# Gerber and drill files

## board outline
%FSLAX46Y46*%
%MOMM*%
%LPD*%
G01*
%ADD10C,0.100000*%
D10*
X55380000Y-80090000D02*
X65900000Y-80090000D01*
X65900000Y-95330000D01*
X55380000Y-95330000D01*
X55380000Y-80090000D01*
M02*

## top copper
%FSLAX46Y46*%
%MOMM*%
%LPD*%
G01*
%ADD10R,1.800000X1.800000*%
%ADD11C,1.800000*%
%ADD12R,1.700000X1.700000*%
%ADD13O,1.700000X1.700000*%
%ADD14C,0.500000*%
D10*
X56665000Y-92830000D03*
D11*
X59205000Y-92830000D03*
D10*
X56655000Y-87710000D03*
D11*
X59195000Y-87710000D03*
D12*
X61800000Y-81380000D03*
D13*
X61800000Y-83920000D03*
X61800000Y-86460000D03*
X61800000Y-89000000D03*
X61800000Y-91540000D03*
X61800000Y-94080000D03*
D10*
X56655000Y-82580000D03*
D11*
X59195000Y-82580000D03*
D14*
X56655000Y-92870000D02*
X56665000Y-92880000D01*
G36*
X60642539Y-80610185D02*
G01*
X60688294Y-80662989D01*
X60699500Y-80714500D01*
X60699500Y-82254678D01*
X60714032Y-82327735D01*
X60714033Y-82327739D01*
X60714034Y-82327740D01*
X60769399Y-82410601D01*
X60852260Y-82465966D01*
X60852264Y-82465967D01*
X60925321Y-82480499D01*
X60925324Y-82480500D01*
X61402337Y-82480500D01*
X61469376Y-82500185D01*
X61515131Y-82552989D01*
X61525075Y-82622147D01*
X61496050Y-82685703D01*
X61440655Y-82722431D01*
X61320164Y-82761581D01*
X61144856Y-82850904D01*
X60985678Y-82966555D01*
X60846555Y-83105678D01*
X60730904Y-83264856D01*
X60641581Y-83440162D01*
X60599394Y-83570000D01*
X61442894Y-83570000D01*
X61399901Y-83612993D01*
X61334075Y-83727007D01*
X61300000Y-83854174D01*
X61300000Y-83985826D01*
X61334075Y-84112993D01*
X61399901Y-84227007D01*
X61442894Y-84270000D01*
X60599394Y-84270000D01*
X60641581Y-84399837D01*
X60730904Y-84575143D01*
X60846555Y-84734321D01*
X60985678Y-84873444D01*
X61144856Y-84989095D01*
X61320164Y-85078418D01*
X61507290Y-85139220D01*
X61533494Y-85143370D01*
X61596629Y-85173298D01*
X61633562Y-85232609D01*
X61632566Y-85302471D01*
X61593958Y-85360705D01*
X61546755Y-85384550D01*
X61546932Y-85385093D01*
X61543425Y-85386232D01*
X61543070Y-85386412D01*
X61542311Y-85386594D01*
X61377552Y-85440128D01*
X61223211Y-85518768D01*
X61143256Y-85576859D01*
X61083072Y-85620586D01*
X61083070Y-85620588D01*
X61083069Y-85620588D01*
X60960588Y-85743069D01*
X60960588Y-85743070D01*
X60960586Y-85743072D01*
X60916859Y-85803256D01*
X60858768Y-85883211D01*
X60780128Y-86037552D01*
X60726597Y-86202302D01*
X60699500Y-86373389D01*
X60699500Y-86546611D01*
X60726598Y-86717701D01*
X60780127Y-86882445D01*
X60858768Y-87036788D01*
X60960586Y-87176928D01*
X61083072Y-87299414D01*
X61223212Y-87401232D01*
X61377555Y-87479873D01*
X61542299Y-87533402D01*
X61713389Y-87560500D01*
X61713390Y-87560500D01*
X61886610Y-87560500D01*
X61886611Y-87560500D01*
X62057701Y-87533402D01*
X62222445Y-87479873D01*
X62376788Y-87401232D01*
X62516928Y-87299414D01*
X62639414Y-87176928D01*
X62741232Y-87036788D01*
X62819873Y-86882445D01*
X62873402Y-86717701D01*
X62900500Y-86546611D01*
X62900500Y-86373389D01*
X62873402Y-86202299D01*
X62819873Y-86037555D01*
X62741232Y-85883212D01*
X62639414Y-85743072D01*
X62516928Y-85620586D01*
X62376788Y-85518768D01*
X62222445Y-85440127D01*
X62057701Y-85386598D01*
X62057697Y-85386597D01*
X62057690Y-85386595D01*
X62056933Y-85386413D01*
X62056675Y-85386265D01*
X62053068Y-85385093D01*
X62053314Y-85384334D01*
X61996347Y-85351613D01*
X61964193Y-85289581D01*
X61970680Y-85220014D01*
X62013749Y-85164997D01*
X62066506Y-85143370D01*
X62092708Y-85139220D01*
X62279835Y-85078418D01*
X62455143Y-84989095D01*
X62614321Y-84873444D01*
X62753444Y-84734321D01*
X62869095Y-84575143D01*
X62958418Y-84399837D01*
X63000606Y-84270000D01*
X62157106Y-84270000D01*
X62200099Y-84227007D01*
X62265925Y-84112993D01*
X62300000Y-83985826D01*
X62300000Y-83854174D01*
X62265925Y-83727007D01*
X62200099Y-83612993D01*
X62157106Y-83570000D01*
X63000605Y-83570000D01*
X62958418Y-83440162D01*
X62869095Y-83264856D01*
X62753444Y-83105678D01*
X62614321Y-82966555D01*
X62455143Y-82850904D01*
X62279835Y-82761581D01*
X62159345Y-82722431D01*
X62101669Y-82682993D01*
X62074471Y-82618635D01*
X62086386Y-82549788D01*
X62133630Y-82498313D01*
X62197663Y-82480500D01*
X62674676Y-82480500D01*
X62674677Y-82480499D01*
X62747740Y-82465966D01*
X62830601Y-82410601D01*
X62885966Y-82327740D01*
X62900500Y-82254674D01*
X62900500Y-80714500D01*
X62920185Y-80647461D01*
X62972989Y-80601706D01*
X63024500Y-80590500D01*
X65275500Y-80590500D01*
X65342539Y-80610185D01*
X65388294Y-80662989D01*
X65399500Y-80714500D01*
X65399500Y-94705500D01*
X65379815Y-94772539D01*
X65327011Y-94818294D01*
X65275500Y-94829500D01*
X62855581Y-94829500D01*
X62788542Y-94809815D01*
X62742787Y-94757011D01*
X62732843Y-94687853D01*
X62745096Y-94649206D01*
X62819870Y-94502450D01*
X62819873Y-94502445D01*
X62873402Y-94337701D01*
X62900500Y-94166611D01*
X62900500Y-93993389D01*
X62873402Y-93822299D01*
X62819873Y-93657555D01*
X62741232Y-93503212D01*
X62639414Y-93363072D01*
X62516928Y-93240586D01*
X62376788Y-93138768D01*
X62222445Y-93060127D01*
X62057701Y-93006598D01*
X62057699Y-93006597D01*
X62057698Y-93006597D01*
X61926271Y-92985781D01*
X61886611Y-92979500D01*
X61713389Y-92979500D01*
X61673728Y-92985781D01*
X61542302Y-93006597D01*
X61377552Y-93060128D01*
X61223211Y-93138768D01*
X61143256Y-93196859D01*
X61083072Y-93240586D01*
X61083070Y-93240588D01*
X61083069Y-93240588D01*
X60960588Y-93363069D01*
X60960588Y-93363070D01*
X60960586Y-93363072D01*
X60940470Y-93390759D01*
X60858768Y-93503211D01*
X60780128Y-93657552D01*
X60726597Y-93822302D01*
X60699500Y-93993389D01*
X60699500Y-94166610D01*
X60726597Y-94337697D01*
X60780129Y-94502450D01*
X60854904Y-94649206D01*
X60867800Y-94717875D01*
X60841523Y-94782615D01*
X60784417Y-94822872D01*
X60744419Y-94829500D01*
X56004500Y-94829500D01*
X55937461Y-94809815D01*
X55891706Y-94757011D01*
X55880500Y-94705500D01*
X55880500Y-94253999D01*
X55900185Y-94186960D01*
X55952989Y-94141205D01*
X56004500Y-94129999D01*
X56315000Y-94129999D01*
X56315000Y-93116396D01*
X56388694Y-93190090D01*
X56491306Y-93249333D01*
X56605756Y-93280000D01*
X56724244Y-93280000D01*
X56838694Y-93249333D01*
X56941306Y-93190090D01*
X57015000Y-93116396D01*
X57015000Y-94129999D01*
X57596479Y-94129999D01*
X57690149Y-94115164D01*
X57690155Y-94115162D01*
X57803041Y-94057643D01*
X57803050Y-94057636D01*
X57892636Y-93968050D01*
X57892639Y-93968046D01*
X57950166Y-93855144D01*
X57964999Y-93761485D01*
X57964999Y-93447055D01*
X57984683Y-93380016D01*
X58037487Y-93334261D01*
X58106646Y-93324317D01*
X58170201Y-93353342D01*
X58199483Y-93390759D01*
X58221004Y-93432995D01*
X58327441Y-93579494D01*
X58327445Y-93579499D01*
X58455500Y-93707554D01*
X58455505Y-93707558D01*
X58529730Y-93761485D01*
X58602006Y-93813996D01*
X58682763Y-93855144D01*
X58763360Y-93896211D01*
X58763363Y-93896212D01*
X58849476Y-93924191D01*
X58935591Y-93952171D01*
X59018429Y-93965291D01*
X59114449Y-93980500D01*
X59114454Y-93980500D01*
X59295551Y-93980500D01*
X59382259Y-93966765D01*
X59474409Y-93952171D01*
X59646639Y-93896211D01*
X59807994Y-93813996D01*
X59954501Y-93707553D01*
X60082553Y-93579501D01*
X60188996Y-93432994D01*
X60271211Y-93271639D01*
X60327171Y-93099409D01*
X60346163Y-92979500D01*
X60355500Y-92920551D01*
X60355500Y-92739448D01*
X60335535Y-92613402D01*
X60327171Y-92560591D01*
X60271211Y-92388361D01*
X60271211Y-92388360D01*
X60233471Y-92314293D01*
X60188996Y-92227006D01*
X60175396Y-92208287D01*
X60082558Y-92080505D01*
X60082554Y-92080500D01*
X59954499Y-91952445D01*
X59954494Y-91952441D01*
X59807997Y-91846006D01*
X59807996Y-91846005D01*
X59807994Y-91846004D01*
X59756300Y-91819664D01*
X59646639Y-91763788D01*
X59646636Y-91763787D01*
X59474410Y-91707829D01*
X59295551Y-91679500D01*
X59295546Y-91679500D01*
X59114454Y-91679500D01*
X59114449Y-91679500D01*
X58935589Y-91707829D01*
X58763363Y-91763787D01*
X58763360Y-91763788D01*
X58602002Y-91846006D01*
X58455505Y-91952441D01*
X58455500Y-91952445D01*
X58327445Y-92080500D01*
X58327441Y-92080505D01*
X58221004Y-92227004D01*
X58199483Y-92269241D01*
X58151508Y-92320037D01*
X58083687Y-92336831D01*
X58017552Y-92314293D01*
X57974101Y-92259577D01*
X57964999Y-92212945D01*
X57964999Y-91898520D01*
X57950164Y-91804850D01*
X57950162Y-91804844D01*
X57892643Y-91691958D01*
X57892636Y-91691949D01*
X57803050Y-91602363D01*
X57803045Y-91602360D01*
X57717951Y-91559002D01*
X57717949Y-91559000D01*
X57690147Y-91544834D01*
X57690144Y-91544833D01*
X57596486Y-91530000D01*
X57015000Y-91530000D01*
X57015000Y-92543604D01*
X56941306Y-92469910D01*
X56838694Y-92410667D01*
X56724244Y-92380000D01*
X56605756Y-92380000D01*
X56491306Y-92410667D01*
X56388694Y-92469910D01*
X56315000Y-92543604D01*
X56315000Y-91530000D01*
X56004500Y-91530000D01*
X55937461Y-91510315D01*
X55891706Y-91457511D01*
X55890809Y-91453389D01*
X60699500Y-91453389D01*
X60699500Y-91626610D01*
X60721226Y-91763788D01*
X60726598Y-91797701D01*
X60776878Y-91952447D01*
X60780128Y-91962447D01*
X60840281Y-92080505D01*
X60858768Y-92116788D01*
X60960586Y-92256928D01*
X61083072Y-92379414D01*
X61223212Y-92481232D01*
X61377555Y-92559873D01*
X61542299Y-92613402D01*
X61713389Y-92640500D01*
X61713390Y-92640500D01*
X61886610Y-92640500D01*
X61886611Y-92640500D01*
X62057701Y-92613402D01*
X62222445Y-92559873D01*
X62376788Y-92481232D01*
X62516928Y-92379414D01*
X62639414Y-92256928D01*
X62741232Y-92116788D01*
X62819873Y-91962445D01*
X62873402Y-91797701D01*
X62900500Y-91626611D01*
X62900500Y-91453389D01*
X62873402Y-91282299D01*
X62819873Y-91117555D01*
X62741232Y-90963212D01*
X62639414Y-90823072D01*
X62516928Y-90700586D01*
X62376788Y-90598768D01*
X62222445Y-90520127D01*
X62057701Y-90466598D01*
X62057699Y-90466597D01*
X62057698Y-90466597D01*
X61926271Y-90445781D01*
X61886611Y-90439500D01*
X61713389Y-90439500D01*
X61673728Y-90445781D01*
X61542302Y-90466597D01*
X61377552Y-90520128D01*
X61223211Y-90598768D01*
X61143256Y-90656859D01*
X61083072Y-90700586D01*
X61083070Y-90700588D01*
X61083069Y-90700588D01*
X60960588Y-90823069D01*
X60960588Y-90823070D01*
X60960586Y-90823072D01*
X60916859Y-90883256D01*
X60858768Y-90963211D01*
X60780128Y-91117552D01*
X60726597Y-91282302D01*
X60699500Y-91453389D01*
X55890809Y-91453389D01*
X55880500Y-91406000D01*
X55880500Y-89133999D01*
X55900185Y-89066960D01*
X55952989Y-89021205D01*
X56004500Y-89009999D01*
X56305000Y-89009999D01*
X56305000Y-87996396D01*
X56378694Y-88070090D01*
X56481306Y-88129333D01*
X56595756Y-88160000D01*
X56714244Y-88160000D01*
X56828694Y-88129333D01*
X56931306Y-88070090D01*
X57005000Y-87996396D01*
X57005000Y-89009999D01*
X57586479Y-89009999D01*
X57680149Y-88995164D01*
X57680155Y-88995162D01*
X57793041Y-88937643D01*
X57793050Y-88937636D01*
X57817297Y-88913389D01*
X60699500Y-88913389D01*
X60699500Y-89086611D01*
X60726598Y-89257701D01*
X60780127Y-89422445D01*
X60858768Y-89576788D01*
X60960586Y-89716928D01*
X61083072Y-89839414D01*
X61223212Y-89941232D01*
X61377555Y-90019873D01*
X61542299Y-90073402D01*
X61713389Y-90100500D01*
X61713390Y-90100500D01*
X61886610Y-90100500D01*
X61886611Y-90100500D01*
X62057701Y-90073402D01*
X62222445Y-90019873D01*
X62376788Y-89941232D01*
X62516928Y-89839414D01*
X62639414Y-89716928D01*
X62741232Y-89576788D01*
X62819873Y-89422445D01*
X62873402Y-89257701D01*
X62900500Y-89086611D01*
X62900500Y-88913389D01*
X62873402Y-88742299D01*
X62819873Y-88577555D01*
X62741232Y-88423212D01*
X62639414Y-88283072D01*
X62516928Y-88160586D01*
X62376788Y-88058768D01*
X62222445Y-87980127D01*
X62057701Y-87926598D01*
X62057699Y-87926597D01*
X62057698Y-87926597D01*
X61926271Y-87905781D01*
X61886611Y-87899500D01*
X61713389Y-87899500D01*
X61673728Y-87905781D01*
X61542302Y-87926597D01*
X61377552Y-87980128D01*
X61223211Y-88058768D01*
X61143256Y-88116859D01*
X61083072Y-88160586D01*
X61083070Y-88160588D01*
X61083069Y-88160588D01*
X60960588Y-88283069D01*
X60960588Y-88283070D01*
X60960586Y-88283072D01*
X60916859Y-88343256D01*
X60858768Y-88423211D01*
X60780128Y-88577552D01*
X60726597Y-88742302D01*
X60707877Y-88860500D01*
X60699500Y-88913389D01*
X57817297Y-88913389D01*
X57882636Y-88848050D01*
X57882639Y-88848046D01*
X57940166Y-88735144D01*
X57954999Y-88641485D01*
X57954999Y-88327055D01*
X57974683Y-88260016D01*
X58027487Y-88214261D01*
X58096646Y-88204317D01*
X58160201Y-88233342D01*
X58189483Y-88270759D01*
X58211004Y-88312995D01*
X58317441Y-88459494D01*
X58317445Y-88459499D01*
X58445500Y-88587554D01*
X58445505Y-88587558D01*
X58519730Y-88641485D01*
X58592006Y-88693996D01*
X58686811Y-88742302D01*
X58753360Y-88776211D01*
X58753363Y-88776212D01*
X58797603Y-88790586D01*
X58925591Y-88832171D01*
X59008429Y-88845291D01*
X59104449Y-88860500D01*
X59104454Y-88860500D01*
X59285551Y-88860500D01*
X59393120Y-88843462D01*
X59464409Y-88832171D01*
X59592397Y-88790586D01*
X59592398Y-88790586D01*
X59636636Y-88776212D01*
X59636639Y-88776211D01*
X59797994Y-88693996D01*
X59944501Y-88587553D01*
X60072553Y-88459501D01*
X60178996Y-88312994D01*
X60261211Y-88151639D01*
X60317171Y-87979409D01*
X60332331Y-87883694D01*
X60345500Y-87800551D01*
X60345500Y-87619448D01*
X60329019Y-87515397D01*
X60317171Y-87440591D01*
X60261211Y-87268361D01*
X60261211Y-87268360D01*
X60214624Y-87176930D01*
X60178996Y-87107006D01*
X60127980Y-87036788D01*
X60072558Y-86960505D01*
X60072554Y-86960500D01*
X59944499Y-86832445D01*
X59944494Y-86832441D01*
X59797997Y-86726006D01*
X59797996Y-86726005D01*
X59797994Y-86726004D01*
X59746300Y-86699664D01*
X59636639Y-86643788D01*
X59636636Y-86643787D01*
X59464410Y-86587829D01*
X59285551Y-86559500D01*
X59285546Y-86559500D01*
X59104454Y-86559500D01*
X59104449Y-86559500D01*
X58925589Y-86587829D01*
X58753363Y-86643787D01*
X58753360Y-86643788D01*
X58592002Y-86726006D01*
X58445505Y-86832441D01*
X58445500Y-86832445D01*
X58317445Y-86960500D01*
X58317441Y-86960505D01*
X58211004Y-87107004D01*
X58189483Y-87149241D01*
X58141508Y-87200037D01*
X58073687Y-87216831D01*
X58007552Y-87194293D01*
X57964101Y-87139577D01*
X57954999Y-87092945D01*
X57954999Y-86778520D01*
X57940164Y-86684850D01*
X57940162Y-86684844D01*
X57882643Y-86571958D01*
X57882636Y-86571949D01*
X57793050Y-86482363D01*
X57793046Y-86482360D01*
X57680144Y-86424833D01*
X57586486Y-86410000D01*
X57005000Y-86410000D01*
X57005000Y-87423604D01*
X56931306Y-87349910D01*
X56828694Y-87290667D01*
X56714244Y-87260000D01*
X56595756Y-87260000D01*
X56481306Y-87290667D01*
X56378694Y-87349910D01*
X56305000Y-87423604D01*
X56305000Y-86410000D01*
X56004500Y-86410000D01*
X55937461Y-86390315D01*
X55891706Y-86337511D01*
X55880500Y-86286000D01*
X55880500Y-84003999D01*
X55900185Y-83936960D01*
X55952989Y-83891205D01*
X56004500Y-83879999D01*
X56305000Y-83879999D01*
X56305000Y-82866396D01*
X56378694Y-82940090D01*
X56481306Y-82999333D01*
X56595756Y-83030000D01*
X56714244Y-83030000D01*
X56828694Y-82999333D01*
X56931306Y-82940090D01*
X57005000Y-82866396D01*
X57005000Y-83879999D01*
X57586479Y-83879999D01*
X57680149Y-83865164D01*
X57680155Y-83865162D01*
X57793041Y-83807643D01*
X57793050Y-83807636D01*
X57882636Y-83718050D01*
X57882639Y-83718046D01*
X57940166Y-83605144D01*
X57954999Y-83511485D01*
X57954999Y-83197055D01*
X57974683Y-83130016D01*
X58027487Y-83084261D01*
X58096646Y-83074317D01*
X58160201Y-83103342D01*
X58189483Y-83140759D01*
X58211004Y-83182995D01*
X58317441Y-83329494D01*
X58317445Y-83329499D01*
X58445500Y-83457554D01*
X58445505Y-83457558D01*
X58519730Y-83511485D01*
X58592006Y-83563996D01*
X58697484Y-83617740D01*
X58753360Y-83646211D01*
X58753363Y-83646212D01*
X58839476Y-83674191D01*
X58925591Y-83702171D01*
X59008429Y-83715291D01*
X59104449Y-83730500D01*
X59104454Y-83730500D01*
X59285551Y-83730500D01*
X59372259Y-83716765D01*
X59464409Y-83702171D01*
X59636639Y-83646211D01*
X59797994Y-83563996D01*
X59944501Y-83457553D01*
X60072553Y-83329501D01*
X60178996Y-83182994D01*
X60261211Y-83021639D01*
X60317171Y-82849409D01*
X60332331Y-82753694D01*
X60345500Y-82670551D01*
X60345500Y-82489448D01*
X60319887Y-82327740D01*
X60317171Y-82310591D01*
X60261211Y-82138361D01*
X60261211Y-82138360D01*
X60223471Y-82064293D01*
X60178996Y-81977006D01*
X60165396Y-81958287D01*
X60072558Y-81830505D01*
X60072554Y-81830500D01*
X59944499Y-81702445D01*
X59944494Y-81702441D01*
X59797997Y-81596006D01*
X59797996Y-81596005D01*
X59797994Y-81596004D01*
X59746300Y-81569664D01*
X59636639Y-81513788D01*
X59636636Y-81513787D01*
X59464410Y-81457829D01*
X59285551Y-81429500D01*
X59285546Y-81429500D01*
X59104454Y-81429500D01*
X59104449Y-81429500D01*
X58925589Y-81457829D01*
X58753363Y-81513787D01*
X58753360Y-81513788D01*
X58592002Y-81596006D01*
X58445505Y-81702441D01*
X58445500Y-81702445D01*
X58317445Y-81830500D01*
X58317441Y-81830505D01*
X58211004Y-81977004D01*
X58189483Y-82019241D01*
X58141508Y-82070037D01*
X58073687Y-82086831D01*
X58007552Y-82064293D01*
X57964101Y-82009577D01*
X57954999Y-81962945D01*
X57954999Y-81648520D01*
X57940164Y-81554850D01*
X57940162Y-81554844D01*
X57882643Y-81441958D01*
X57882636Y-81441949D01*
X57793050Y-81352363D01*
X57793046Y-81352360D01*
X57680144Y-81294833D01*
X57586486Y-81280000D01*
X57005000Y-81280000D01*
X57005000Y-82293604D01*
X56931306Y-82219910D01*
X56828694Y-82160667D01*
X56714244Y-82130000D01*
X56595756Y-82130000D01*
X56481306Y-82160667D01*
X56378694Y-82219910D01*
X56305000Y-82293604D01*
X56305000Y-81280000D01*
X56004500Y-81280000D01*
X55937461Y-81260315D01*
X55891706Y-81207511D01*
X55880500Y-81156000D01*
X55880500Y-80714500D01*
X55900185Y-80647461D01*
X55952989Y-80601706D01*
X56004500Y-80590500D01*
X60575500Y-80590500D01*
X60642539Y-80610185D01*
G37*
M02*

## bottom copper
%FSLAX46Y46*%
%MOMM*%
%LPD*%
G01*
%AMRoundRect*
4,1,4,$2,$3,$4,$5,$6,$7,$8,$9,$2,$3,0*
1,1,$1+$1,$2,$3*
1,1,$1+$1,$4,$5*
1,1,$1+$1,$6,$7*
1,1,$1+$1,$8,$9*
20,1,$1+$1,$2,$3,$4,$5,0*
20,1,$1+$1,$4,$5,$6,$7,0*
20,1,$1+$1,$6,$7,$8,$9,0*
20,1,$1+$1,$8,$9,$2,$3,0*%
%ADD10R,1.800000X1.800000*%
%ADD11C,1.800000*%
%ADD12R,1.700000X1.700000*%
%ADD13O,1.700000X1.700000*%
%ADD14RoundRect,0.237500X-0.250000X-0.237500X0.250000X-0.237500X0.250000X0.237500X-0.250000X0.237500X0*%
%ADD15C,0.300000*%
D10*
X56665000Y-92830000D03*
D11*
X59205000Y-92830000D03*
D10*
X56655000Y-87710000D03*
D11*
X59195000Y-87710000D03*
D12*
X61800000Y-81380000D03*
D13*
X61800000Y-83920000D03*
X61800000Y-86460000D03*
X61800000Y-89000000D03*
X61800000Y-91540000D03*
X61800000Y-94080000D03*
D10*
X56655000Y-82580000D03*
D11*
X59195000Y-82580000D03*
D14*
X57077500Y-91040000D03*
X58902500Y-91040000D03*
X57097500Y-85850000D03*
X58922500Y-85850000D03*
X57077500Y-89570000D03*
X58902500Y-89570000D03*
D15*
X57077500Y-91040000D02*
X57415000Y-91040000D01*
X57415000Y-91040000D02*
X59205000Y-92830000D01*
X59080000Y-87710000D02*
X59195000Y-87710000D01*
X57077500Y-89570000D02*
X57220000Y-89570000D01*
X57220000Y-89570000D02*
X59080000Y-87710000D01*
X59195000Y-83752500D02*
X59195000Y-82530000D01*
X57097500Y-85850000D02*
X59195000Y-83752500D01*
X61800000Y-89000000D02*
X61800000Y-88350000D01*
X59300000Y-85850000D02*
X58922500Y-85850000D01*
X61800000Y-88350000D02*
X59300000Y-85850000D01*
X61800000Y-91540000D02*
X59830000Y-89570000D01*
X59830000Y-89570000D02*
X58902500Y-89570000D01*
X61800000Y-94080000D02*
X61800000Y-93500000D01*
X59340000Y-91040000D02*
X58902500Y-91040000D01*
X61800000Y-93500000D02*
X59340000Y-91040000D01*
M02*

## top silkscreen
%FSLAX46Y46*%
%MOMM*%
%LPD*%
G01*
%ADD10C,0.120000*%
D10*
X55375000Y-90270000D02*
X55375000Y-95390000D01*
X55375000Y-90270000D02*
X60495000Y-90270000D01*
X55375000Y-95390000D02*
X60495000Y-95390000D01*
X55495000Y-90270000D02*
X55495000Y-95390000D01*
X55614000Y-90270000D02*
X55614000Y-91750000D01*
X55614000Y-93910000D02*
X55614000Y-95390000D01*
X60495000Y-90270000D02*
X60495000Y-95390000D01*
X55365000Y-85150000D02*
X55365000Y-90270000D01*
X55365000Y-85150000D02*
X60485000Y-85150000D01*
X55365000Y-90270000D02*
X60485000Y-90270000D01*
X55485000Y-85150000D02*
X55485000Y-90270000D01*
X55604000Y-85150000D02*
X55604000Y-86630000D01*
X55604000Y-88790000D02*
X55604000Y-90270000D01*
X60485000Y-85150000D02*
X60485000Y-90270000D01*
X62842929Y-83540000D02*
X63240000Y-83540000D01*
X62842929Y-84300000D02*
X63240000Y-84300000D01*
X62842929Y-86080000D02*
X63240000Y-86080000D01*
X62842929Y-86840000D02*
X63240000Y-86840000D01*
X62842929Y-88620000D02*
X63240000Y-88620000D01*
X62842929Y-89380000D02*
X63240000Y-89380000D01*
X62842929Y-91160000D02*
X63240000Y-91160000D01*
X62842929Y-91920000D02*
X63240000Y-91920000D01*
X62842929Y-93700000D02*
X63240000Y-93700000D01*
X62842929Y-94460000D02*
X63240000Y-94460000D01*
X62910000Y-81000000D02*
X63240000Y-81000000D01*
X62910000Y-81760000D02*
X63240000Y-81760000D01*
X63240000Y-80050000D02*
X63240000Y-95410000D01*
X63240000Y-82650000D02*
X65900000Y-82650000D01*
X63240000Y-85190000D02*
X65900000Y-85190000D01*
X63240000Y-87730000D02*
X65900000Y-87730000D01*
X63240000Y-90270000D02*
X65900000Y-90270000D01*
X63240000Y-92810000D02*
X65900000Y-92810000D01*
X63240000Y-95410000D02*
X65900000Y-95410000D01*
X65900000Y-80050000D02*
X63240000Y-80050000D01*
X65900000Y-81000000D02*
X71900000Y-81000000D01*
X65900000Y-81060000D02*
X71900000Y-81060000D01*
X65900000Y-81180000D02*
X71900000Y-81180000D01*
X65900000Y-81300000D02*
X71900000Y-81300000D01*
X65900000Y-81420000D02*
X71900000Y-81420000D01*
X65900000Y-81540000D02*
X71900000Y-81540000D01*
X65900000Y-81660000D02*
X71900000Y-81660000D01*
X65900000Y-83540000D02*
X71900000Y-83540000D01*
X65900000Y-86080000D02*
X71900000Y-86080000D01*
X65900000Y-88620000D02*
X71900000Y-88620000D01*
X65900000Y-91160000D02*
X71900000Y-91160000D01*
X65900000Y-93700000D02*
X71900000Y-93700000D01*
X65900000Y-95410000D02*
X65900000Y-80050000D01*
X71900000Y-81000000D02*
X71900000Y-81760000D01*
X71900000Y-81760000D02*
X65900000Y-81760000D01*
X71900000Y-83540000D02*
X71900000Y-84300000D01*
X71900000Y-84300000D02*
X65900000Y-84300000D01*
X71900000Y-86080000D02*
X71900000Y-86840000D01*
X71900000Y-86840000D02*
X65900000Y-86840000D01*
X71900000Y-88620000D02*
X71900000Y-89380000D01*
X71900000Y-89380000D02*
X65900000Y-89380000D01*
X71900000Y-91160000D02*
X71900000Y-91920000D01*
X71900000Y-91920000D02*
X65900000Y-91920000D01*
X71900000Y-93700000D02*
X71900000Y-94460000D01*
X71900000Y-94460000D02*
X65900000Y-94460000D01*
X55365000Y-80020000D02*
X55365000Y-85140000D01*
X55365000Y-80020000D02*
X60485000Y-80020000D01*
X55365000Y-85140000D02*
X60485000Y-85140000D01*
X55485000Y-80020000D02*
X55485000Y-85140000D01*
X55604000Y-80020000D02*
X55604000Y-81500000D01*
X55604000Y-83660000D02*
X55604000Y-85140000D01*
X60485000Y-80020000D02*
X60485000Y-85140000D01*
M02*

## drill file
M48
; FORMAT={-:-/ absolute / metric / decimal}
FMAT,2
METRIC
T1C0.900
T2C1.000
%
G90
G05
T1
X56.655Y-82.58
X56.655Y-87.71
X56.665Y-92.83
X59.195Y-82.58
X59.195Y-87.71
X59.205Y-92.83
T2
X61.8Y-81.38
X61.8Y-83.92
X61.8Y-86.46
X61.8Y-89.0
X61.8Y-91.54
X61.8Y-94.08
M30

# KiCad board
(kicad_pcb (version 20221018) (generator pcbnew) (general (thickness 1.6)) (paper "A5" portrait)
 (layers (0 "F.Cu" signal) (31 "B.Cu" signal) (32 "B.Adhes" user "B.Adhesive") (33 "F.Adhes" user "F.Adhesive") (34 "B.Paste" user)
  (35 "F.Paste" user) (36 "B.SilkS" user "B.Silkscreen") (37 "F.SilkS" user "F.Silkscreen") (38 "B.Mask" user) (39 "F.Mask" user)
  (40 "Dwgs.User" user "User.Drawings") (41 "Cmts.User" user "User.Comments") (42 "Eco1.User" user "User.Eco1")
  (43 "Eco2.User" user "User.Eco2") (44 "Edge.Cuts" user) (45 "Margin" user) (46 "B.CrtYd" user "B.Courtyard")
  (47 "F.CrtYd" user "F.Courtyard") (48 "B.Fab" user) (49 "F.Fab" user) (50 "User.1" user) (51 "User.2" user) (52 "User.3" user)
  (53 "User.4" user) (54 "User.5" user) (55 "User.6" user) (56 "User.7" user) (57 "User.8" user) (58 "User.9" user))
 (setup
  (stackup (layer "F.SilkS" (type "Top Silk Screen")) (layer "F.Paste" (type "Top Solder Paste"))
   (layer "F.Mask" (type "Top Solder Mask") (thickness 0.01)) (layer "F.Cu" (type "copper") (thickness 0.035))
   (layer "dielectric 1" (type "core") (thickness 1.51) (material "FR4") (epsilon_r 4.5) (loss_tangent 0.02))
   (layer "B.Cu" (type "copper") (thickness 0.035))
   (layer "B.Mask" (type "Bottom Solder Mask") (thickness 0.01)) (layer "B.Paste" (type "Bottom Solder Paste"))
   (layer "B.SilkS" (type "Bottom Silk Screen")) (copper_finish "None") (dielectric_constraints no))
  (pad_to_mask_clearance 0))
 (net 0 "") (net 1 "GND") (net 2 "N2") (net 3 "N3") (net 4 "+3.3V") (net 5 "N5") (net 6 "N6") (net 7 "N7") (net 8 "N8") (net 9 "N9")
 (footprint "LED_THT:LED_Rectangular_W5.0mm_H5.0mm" (layer "F.Cu") (at 56.665 92.83)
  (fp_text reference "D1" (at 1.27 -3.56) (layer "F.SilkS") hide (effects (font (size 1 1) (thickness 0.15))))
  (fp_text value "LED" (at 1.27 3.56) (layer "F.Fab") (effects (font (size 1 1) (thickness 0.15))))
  (fp_line (start -1.29 -2.56) (end -1.29 2.56) (stroke (width 0.12) (type solid)) (layer "F.SilkS"))
  (fp_line (start -1.29 -2.56) (end 3.83 -2.56) (stroke (width 0.12) (type solid)) (layer "F.SilkS"))
  (fp_line (start -1.29 2.56) (end 3.83 2.56) (stroke (width 0.12) (type solid)) (layer "F.SilkS"))
  (fp_line (start -1.17 -2.56) (end -1.17 2.56) (stroke (width 0.12) (type solid)) (layer "F.SilkS"))
  (fp_line (start -1.051 -2.56) (end -1.051 -1.08) (stroke (width 0.12) (type solid)) (layer "F.SilkS"))
  (fp_line (start -1.051 1.08) (end -1.051 2.56) (stroke (width 0.12) (type solid)) (layer "F.SilkS"))
  (fp_line (start 3.83 -2.56) (end 3.83 2.56) (stroke (width 0.12) (type solid)) (layer "F.SilkS"))
  (pad "1" thru_hole rect (at 0 0) (size 1.8 1.8) (drill 0.9) (layers "*.Cu" "*.Mask") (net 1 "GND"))
  (pad "2" thru_hole circle (at 2.54 0) (size 1.8 1.8) (drill 0.9) (layers "*.Cu" "*.Mask") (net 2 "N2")))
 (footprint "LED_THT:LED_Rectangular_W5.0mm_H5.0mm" (layer "F.Cu") (at 56.655 87.71)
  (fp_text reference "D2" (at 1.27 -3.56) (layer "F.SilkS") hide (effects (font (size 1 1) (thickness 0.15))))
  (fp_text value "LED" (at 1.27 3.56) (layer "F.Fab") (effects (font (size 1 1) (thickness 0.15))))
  (fp_line (start -1.29 -2.56) (end -1.29 2.56) (stroke (width 0.12) (type solid)) (layer "F.SilkS"))
  (fp_line (start -1.29 -2.56) (end 3.83 -2.56) (stroke (width 0.12) (type solid)) (layer "F.SilkS"))
  (fp_line (start -1.29 2.56) (end 3.83 2.56) (stroke (width 0.12) (type solid)) (layer "F.SilkS"))
  (fp_line (start -1.17 -2.56) (end -1.17 2.56) (stroke (width 0.12) (type solid)) (layer "F.SilkS"))
  (fp_line (start -1.051 -2.56) (end -1.051 -1.08) (stroke (width 0.12) (type solid)) (layer "F.SilkS"))
  (fp_line (start -1.051 1.08) (end -1.051 2.56) (stroke (width 0.12) (type solid)) (layer "F.SilkS"))
  (fp_line (start 3.83 -2.56) (end 3.83 2.56) (stroke (width 0.12) (type solid)) (layer "F.SilkS"))
  (pad "1" thru_hole rect (at 0 0) (size 1.8 1.8) (drill 0.9) (layers "*.Cu" "*.Mask") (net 1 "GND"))
  (pad "2" thru_hole circle (at 2.54 0) (size 1.8 1.8) (drill 0.9) (layers "*.Cu" "*.Mask") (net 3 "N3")))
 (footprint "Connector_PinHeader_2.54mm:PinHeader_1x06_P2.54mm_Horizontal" (layer "F.Cu") (at 61.8 81.38)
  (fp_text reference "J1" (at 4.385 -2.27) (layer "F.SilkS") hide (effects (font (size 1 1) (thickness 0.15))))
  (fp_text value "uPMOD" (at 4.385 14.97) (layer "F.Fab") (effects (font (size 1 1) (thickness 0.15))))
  (fp_line (start 1.042929 2.16) (end 1.44 2.16) (stroke (width 0.12) (type solid)) (layer "F.SilkS"))
  (fp_line (start 1.042929 2.92) (end 1.44 2.92) (stroke (width 0.12) (type solid)) (layer "F.SilkS"))
  (fp_line (start 1.042929 4.7) (end 1.44 4.7) (stroke (width 0.12) (type solid)) (layer "F.SilkS"))
  (fp_line (start 1.042929 5.46) (end 1.44 5.46) (stroke (width 0.12) (type solid)) (layer "F.SilkS"))
  (fp_line (start 1.042929 7.24) (end 1.44 7.24) (stroke (width 0.12) (type solid)) (layer "F.SilkS"))
  (fp_line (start 1.042929 8) (end 1.44 8) (stroke (width 0.12) (type solid)) (layer "F.SilkS"))
  (fp_line (start 1.042929 9.78) (end 1.44 9.78) (stroke (width 0.12) (type solid)) (layer "F.SilkS"))
  (fp_line (start 1.042929 10.54) (end 1.44 10.54) (stroke (width 0.12) (type solid)) (layer "F.SilkS"))
  (fp_line (start 1.042929 12.32) (end 1.44 12.32) (stroke (width 0.12) (type solid)) (layer "F.SilkS"))
  (fp_line (start 1.042929 13.08) (end 1.44 13.08) (stroke (width 0.12) (type solid)) (layer "F.SilkS"))
  (fp_line (start 1.11 -0.38) (end 1.44 -0.38) (stroke (width 0.12) (type solid)) (layer "F.SilkS"))
  (fp_line (start 1.11 0.38) (end 1.44 0.38) (stroke (width 0.12) (type solid)) (layer "F.SilkS"))
  (fp_line (start 1.44 -1.33) (end 1.44 14.03) (stroke (width 0.12) (type solid)) (layer "F.SilkS"))
  (fp_line (start 1.44 1.27) (end 4.1 1.27) (stroke (width 0.12) (type solid)) (layer "F.SilkS"))
  (fp_line (start 1.44 3.81) (end 4.1 3.81) (stroke (width 0.12) (type solid)) (layer "F.SilkS"))
  (fp_line (start 1.44 6.35) (end 4.1 6.35) (stroke (width 0.12) (type solid)) (layer "F.SilkS"))
  (fp_line (start 1.44 8.89) (end 4.1 8.89) (stroke (width 0.12) (type solid)) (layer "F.SilkS"))
  (fp_line (start 1.44 11.43) (end 4.1 11.43) (stroke (width 0.12) (type solid)) (layer "F.SilkS"))
  (fp_line (start 1.44 14.03) (end 4.1 14.03) (stroke (width 0.12) (type solid)) (layer "F.SilkS"))
  (fp_line (start 4.1 -1.33) (end 1.44 -1.33) (stroke (width 0.12) (type solid)) (layer "F.SilkS"))
  (fp_line (start 4.1 -0.38) (end 10.1 -0.38) (stroke (width 0.12) (type solid)) (layer "F.SilkS"))
  (fp_line (start 4.1 -0.32) (end 10.1 -0.32) (stroke (width 0.12) (type solid)) (layer "F.SilkS"))
  (fp_line (start 4.1 -0.2) (end 10.1 -0.2) (stroke (width 0.12) (type solid)) (layer "F.SilkS"))
  (fp_line (start 4.1 -0.08) (end 10.1 -0.08) (stroke (width 0.12) (type solid)) (layer "F.SilkS"))
  (fp_line (start 4.1 0.04) (end 10.1 0.04) (stroke (width 0.12) (type solid)) (layer "F.SilkS"))
  (fp_line (start 4.1 0.16) (end 10.1 0.16) (stroke (width 0.12) (type solid)) (layer "F.SilkS"))
  (fp_line (start 4.1 0.28) (end 10.1 0.28) (stroke (width 0.12) (type solid)) (layer "F.SilkS"))
  (fp_line (start 4.1 2.16) (end 10.1 2.16) (stroke (width 0.12) (type solid)) (layer "F.SilkS"))
  (fp_line (start 4.1 4.7) (end 10.1 4.7) (stroke (width 0.12) (type solid)) (layer "F.SilkS"))
  (fp_line (start 4.1 7.24) (end 10.1 7.24) (stroke (width 0.12) (type solid)) (layer "F.SilkS"))
  (fp_line (start 4.1 9.78) (end 10.1 9.78) (stroke (width 0.12) (type solid)) (layer "F.SilkS"))
  (fp_line (start 4.1 12.32) (end 10.1 12.32) (stroke (width 0.12) (type solid)) (layer "F.SilkS"))
  (fp_line (start 4.1 14.03) (end 4.1 -1.33) (stroke (width 0.12) (type solid)) (layer "F.SilkS"))
  (fp_line (start 10.1 -0.38) (end 10.1 0.38) (stroke (width 0.12) (type solid)) (layer "F.SilkS"))
  (fp_line (start 10.1 0.38) (end 4.1 0.38) (stroke (width 0.12) (type solid)) (layer "F.SilkS"))
  (fp_line (start 10.1 2.16) (end 10.1 2.92) (stroke (width 0.12) (type solid)) (layer "F.SilkS"))
  (fp_line (start 10.1 2.92) (end 4.1 2.92) (stroke (width 0.12) (type solid)) (layer "F.SilkS"))
  (fp_line (start 10.1 4.7) (end 10.1 5.46) (stroke (width 0.12) (type solid)) (layer "F.SilkS"))
  (fp_line (start 10.1 5.46) (end 4.1 5.46) (stroke (width 0.12) (type solid)) (layer "F.SilkS"))
  (fp_line (start 10.1 7.24) (end 10.1 8) (stroke (width 0.12) (type solid)) (layer "F.SilkS"))
  (fp_line (start 10.1 8) (end 4.1 8) (stroke (width 0.12) (type solid)) (layer "F.SilkS"))
  (fp_line (start 10.1 9.78) (end 10.1 10.54) (stroke (width 0.12) (type solid)) (layer "F.SilkS"))
  (fp_line (start 10.1 10.54) (end 4.1 10.54) (stroke (width 0.12) (type solid)) (layer "F.SilkS"))
  (fp_line (start 10.1 12.32) (end 10.1 13.08) (stroke (width 0.12) (type solid)) (layer "F.SilkS"))
  (fp_line (start 10.1 13.08) (end 4.1 13.08) (stroke (width 0.12) (type solid)) (layer "F.SilkS"))
  (pad "1" thru_hole rect (at 0 0) (size 1.7 1.7) (drill 1) (layers "*.Cu" "*.Mask") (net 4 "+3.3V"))
  (pad "2" thru_hole oval (at 0 2.54) (size 1.7 1.7) (drill 1) (layers "*.Cu" "*.Mask") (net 1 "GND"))
  (pad "3" thru_hole oval (at 0 5.08) (size 1.7 1.7) (drill 1) (layers "*.Cu" "*.Mask") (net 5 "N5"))
  (pad "4" thru_hole oval (at 0 7.62) (size 1.7 1.7) (drill 1) (layers "*.Cu" "*.Mask") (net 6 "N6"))
  (pad "5" thru_hole oval (at 0 10.16) (size 1.7 1.7) (drill 1) (layers "*.Cu" "*.Mask") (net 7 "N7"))
  (pad "6" thru_hole oval (at 0 12.7) (size 1.7 1.7) (drill 1) (layers "*.Cu" "*.Mask") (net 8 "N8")))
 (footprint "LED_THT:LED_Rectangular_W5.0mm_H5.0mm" (layer "F.Cu") (at 56.655 82.58)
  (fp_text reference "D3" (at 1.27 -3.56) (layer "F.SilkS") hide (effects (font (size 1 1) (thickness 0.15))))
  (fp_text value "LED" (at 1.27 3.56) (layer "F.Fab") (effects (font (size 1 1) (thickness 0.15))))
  (fp_line (start -1.29 -2.56) (end -1.29 2.56) (stroke (width 0.12) (type solid)) (layer "F.SilkS"))
  (fp_line (start -1.29 -2.56) (end 3.83 -2.56) (stroke (width 0.12) (type solid)) (layer "F.SilkS"))
  (fp_line (start -1.29 2.56) (end 3.83 2.56) (stroke (width 0.12) (type solid)) (layer "F.SilkS"))
  (fp_line (start -1.17 -2.56) (end -1.17 2.56) (stroke (width 0.12) (type solid)) (layer "F.SilkS"))
  (fp_line (start -1.051 -2.56) (end -1.051 -1.08) (stroke (width 0.12) (type solid)) (layer "F.SilkS"))
  (fp_line (start -1.051 1.08) (end -1.051 2.56) (stroke (width 0.12) (type solid)) (layer "F.SilkS"))
  (fp_line (start 3.83 -2.56) (end 3.83 2.56) (stroke (width 0.12) (type solid)) (layer "F.SilkS"))
  (pad "1" thru_hole rect (at 0 0) (size 1.8 1.8) (drill 0.9) (layers "*.Cu" "*.Mask") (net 1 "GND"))
  (pad "2" thru_hole circle (at 2.54 0) (size 1.8 1.8) (drill 0.9) (layers "*.Cu" "*.Mask") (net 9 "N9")))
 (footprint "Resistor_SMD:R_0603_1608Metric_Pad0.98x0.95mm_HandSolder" (layer "B.Cu") (at 57.99 91.04)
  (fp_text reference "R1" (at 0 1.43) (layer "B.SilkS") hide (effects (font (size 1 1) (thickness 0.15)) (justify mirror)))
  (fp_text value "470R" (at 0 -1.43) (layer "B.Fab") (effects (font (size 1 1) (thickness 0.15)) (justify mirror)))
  (pad "1" smd roundrect (at -0.9125 0) (size 0.975 0.95) (layers "B.Cu" "B.Paste" "B.Mask") (roundrect_rratio 0.25) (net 2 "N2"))
  (pad "2" smd roundrect (at 0.9125 0) (size 0.975 0.95) (layers "B.Cu" "B.Paste" "B.Mask") (roundrect_rratio 0.25) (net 8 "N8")))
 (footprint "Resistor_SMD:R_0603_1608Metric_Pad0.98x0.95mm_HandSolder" (layer "B.Cu") (at 58.01 85.85)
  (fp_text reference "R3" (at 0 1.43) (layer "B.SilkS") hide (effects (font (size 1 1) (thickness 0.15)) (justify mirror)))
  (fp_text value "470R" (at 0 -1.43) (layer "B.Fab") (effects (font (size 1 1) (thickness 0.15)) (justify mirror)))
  (pad "1" smd roundrect (at -0.9125 0) (size 0.975 0.95) (layers "B.Cu" "B.Paste" "B.Mask") (roundrect_rratio 0.25) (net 9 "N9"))
  (pad "2" smd roundrect (at 0.9125 0) (size 0.975 0.95) (layers "B.Cu" "B.Paste" "B.Mask") (roundrect_rratio 0.25) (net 6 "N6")))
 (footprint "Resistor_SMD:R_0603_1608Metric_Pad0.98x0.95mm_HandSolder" (layer "B.Cu") (at 57.99 89.57)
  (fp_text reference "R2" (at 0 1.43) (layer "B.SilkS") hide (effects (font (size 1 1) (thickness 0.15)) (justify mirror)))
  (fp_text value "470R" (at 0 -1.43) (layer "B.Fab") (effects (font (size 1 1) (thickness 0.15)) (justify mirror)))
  (pad "1" smd roundrect (at -0.9125 0) (size 0.975 0.95) (layers "B.Cu" "B.Paste" "B.Mask") (roundrect_rratio 0.25) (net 3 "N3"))
  (pad "2" smd roundrect (at 0.9125 0) (size 0.975 0.95) (layers "B.Cu" "B.Paste" "B.Mask") (roundrect_rratio 0.25) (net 7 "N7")))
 (gr_rect (start 55.38 80.09) (end 65.9 95.33) (stroke (width 0.1) (type default)) (fill none) (layer "Edge.Cuts"))
 (segment (start 56.655 92.87) (end 56.665 92.88) (width 0.5) (layer "F.Cu") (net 1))
 (segment (start 57.0775 91.04) (end 57.415 91.04) (width 0.3) (layer "B.Cu") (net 2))
 (segment (start 57.415 91.04) (end 59.205 92.83) (width 0.3) (layer "B.Cu") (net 2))
 (segment (start 59.08 87.71) (end 59.195 87.71) (width 0.3) (layer "B.Cu") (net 3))
 (segment (start 57.0775 89.57) (end 57.22 89.57) (width 0.3) (layer "B.Cu") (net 3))
 (segment (start 57.22 89.57) (end 59.08 87.71) (width 0.3) (layer "B.Cu") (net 3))
 (segment (start 59.195 83.7525) (end 59.195 82.53) (width 0.3) (layer "B.Cu") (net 9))
 (segment (start 57.0975 85.85) (end 59.195 83.7525) (width 0.3) (layer "B.Cu") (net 9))
 (segment (start 61.8 89) (end 61.8 88.35) (width 0.3) (layer "B.Cu") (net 6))
 (segment (start 59.3 85.85) (end 58.9225 85.85) (width 0.3) (layer "B.Cu") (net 6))
 (segment (start 61.8 88.35) (end 59.3 85.85) (width 0.3) (layer "B.Cu") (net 6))
 (segment (start 61.8 91.54) (end 59.83 89.57) (width 0.3) (layer "B.Cu") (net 7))
 (segment (start 59.83 89.57) (end 58.9025 89.57) (width 0.3) (layer "B.Cu") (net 7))
 (segment (start 61.8 94.08) (end 61.8 93.5) (width 0.3) (layer "B.Cu") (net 8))
 (segment (start 59.34 91.04) (end 58.9025 91.04) (width 0.3) (layer "B.Cu") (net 8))
 (segment (start 61.8 93.5) (end 59.34 91.04) (width 0.3) (layer "B.Cu") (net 8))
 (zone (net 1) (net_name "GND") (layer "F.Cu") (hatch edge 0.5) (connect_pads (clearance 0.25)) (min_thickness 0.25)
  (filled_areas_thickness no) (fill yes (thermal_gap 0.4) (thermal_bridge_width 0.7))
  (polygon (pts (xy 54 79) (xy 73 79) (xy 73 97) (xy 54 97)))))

